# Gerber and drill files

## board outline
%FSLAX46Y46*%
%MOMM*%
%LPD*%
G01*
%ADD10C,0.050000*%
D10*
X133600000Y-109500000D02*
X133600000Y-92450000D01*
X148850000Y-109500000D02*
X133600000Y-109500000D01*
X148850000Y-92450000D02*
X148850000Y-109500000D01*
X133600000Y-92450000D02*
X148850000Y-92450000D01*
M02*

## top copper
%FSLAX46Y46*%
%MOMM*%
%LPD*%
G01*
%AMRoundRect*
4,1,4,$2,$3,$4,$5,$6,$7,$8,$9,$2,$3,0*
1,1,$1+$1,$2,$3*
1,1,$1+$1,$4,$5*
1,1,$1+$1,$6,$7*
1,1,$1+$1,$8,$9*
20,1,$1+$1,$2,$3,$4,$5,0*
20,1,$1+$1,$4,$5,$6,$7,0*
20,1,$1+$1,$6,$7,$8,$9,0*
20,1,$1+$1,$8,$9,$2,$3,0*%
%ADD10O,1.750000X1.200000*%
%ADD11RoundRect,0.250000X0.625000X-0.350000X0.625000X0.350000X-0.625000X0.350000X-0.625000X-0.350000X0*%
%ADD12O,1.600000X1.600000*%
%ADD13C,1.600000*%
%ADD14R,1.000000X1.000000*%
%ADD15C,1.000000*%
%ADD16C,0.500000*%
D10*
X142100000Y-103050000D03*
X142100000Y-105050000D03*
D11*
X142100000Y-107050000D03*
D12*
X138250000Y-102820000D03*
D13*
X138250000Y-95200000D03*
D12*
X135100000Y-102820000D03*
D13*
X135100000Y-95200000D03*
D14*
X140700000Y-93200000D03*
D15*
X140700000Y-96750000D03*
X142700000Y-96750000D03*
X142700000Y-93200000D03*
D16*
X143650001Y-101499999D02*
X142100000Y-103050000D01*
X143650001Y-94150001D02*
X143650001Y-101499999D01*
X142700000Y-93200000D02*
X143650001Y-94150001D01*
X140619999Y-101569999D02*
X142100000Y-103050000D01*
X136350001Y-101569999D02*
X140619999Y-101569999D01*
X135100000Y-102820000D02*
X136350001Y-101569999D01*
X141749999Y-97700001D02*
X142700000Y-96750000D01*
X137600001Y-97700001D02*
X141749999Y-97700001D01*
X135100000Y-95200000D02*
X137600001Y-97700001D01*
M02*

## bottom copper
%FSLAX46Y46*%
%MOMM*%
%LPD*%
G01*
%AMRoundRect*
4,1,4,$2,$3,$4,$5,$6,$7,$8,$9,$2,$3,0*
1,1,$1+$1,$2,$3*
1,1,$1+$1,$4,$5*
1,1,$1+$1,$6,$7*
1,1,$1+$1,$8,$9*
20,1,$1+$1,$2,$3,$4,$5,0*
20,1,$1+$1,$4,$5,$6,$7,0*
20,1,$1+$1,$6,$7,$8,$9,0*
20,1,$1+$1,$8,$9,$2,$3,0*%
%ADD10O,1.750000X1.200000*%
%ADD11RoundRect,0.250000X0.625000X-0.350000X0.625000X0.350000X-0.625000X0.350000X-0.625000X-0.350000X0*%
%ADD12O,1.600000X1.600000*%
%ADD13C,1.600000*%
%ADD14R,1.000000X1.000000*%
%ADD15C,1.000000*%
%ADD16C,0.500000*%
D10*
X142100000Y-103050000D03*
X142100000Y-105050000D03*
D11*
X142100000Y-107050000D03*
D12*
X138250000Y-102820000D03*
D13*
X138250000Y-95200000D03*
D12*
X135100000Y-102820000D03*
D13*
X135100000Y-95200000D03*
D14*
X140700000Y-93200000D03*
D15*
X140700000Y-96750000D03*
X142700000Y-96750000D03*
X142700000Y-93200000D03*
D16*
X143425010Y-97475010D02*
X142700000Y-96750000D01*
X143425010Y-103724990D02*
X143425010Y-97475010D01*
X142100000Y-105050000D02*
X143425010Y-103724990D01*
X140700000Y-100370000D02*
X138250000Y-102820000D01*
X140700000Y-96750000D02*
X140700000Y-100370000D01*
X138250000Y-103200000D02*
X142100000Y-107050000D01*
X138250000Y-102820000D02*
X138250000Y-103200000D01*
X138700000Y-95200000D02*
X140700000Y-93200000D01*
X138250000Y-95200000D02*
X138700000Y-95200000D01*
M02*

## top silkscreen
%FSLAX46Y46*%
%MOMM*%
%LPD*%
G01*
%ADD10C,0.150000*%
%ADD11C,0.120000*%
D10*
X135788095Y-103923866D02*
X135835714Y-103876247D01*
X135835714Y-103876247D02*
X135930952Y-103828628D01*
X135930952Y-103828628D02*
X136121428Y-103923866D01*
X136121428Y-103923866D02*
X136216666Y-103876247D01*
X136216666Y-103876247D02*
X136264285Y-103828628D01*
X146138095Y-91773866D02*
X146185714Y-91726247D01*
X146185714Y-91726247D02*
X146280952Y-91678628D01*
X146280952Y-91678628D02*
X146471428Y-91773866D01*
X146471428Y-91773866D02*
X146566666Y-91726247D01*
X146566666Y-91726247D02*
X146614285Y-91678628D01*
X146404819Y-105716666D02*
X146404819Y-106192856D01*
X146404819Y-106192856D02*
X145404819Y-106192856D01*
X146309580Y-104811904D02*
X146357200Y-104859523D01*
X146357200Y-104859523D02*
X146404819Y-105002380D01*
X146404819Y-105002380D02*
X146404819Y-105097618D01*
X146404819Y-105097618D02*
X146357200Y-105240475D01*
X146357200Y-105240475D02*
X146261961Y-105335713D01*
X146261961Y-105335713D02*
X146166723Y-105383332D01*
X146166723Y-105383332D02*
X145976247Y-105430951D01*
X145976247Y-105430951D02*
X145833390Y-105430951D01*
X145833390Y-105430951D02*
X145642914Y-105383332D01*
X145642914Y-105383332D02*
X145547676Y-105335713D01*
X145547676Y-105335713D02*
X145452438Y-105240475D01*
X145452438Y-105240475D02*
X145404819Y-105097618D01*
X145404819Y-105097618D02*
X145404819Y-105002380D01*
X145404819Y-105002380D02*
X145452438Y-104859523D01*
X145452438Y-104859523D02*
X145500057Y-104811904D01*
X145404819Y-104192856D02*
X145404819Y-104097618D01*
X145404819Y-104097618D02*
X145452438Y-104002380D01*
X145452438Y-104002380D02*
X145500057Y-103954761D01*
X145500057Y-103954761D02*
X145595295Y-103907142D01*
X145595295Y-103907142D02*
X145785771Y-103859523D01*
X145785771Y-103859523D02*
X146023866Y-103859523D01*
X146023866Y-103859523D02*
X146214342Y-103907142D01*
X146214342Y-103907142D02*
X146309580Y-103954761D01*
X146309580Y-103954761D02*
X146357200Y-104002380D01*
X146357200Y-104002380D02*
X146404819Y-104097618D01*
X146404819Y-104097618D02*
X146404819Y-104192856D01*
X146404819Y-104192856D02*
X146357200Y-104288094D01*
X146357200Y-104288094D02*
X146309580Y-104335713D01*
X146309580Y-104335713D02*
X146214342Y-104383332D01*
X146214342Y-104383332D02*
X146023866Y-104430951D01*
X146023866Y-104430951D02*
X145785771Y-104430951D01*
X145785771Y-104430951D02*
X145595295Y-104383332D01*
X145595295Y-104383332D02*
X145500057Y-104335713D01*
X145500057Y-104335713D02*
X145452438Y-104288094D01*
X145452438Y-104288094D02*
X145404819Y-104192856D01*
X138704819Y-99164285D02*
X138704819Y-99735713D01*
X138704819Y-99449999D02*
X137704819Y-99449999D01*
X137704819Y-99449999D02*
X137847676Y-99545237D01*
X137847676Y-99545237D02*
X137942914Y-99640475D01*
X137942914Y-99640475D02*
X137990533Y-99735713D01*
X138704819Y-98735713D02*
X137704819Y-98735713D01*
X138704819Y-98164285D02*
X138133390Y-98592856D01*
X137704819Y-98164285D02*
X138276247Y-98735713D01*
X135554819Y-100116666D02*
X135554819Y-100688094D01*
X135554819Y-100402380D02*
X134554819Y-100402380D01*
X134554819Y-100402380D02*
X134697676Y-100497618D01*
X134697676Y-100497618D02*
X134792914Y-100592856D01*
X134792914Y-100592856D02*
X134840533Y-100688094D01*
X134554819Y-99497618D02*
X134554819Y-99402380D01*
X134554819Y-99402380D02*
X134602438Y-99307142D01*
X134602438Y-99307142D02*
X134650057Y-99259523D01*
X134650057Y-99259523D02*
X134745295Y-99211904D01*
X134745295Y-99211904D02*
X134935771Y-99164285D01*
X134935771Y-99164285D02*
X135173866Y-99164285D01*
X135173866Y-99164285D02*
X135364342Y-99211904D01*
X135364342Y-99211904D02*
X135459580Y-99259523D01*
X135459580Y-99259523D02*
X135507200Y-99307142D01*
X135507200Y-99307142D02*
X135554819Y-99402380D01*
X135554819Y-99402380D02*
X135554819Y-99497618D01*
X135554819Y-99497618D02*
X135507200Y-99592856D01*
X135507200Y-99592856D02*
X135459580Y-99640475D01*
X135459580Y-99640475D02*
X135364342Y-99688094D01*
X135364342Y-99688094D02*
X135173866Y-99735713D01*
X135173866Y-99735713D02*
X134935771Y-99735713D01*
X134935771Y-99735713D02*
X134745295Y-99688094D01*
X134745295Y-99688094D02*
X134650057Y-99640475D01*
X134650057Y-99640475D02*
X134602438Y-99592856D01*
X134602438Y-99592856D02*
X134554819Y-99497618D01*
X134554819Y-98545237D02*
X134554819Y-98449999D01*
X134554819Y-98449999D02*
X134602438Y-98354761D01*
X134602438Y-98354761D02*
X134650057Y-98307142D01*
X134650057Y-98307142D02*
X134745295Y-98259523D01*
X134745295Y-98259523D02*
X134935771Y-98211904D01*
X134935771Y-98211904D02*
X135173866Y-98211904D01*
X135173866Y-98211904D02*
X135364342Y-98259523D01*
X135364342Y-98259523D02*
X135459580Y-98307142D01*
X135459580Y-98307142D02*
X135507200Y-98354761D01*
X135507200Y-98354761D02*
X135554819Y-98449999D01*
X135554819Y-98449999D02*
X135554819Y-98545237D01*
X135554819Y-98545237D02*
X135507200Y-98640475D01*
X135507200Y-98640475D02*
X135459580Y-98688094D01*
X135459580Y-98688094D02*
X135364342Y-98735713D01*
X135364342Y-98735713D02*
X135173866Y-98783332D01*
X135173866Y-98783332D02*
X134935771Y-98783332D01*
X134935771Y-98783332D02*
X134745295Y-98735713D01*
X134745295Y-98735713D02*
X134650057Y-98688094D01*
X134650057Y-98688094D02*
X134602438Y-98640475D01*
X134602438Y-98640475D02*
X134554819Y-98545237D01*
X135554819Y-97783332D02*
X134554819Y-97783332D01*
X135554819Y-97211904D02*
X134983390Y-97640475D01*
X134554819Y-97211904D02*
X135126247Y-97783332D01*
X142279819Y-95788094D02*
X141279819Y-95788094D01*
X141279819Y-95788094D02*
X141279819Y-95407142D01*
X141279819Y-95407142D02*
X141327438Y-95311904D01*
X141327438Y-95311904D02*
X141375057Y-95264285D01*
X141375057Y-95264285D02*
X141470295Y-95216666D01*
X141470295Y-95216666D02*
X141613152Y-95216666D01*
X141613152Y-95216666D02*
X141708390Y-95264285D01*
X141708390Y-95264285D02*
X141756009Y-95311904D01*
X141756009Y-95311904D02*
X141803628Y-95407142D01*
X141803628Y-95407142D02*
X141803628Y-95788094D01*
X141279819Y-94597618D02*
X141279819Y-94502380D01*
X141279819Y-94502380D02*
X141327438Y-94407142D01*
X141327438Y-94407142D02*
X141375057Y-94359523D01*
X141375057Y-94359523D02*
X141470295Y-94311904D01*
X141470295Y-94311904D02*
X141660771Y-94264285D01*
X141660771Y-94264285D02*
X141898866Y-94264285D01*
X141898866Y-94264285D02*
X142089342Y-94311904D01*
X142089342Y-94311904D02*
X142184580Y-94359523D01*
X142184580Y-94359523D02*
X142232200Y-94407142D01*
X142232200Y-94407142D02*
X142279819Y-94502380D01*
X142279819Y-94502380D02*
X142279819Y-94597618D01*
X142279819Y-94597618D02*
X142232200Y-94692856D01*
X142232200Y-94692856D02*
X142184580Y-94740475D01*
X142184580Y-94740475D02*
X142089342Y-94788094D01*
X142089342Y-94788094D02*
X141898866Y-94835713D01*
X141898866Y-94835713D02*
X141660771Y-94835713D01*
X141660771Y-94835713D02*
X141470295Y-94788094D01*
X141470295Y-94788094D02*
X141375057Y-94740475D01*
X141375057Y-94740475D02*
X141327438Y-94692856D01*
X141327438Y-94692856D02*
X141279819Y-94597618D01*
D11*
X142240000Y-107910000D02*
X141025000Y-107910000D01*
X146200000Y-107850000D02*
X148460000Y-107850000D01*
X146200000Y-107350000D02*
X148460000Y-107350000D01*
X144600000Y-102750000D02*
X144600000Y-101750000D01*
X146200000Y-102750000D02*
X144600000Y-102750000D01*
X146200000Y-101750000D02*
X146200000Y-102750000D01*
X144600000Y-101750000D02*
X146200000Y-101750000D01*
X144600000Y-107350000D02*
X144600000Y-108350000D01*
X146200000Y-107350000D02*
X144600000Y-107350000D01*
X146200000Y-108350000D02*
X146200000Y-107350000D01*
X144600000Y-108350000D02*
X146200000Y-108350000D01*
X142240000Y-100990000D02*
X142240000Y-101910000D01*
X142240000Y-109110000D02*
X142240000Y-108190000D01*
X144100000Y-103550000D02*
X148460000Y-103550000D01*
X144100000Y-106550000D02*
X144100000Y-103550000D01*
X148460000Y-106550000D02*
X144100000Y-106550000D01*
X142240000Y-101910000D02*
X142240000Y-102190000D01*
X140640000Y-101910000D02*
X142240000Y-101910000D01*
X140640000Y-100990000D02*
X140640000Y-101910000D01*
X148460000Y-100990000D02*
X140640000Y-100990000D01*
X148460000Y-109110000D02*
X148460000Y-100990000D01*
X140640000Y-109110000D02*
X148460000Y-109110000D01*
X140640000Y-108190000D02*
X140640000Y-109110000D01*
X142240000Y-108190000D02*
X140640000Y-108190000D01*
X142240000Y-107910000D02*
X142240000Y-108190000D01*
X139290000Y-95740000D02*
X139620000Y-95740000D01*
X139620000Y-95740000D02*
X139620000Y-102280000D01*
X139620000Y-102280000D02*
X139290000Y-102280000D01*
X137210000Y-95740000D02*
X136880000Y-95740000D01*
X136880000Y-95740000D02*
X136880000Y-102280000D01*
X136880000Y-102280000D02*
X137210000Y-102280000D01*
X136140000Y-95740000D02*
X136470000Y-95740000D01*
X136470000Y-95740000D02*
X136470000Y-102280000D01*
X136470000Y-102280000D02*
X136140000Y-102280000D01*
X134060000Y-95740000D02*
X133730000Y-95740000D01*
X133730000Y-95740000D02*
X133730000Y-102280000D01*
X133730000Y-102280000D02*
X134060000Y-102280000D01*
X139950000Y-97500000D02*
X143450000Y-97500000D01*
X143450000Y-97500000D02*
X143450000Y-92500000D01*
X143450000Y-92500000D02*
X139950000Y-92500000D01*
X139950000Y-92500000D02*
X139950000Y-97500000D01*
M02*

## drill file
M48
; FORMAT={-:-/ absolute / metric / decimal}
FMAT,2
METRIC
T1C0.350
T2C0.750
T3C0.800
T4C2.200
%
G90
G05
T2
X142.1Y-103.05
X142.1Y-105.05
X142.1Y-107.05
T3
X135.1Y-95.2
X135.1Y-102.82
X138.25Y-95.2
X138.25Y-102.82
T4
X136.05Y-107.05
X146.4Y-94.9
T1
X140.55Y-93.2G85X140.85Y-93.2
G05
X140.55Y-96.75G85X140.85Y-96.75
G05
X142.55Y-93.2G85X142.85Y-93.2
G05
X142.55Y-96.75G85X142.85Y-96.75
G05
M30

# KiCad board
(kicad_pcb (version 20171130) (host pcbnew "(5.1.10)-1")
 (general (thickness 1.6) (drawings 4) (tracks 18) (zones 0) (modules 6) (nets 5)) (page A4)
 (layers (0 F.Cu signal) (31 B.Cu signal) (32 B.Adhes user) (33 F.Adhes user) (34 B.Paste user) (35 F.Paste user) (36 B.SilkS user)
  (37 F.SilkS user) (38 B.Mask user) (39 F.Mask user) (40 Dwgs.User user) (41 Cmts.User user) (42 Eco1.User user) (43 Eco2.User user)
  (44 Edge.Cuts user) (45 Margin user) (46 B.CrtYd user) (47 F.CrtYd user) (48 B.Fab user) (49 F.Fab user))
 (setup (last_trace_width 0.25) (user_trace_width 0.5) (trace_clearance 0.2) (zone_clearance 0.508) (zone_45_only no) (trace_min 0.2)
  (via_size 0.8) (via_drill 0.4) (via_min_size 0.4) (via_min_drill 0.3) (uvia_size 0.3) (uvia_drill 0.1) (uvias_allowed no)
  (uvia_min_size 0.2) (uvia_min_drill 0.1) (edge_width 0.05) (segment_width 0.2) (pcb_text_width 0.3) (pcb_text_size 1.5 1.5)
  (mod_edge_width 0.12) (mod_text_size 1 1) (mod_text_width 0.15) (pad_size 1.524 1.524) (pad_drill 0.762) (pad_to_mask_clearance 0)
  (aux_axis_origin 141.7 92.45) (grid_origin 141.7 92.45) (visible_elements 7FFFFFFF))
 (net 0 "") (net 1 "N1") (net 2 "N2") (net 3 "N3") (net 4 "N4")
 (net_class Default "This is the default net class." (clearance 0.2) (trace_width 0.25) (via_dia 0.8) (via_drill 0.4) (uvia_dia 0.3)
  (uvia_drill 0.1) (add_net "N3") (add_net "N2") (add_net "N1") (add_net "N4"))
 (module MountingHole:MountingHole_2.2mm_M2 (layer F.Cu) (at 136.05 107.05) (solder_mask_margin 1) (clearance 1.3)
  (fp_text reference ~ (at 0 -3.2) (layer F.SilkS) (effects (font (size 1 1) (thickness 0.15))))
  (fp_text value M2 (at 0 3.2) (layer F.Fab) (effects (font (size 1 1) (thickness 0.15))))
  (pad 1 np_thru_hole circle (at 0 0) (size 2.2 2.2) (drill 2.2) (layers *.Cu *.Mask)))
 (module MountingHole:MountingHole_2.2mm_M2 (layer F.Cu) (at 146.4 94.9) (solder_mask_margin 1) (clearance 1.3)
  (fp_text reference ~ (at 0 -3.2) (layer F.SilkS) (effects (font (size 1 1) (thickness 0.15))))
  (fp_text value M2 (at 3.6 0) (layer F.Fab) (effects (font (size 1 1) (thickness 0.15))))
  (pad 1 np_thru_hole circle (at 0 0) (size 2.2 2.2) (drill 2.2) (layers *.Cu *.Mask)))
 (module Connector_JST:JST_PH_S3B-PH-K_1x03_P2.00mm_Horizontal (layer F.Cu) (at 142.1 107.05 90)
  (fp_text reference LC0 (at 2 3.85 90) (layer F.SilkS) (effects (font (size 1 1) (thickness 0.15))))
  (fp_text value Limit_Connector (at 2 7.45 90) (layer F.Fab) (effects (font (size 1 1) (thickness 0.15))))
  (fp_line (start -0.86 0.14) (end -0.86 -1.075) (layer F.SilkS) (width 0.12))
  (fp_line (start -0.8 4.1) (end -0.8 6.36) (layer F.SilkS) (width 0.12))
  (fp_line (start -0.3 4.1) (end -0.3 6.36) (layer F.SilkS) (width 0.12))
  (fp_line (start 4.3 2.5) (end 5.3 2.5) (layer F.SilkS) (width 0.12))
  (fp_line (start 4.3 4.1) (end 4.3 2.5) (layer F.SilkS) (width 0.12))
  (fp_line (start 5.3 4.1) (end 4.3 4.1) (layer F.SilkS) (width 0.12))
  (fp_line (start 5.3 2.5) (end 5.3 4.1) (layer F.SilkS) (width 0.12))
  (fp_line (start -0.3 2.5) (end -1.3 2.5) (layer F.SilkS) (width 0.12))
  (fp_line (start -0.3 4.1) (end -0.3 2.5) (layer F.SilkS) (width 0.12))
  (fp_line (start -1.3 4.1) (end -0.3 4.1) (layer F.SilkS) (width 0.12))
  (fp_line (start -1.3 2.5) (end -1.3 4.1) (layer F.SilkS) (width 0.12))
  (fp_line (start 6.06 0.14) (end 5.14 0.14) (layer F.SilkS) (width 0.12))
  (fp_line (start -2.06 0.14) (end -1.14 0.14) (layer F.SilkS) (width 0.12))
  (fp_line (start 3.5 2) (end 3.5 6.36) (layer F.SilkS) (width 0.12))
  (fp_line (start 0.5 2) (end 3.5 2) (layer F.SilkS) (width 0.12))
  (fp_line (start 0.5 6.36) (end 0.5 2) (layer F.SilkS) (width 0.12))
  (fp_line (start 5.14 0.14) (end 4.86 0.14) (layer F.SilkS) (width 0.12))
  (fp_line (start 5.14 -1.46) (end 5.14 0.14) (layer F.SilkS) (width 0.12))
  (fp_line (start 6.06 -1.46) (end 5.14 -1.46) (layer F.SilkS) (width 0.12))
  (fp_line (start 6.06 6.36) (end 6.06 -1.46) (layer F.SilkS) (width 0.12))
  (fp_line (start -2.06 6.36) (end 6.06 6.36) (layer F.SilkS) (width 0.12))
  (fp_line (start -2.06 -1.46) (end -2.06 6.36) (layer F.SilkS) (width 0.12))
  (fp_line (start -1.14 -1.46) (end -2.06 -1.46) (layer F.SilkS) (width 0.12))
  (fp_line (start -1.14 0.14) (end -1.14 -1.46) (layer F.SilkS) (width 0.12))
  (fp_line (start -0.86 0.14) (end -1.14 0.14) (layer F.SilkS) (width 0.12))
  (pad 3 thru_hole oval (at 4 0 90) (size 1.2 1.75) (drill 0.75) (layers *.Cu *.Mask) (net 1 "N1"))
  (pad 2 thru_hole oval (at 2 0 90) (size 1.2 1.75) (drill 0.75) (layers *.Cu *.Mask) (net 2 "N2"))
  (pad 1 thru_hole roundrect (at 0 0 90) (size 1.2 1.75) (drill 0.75) (layers *.Cu *.Mask) (roundrect_rratio 0.208333) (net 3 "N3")))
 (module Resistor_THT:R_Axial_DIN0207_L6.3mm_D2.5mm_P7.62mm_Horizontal (layer F.Cu) (at 138.25 95.2 270)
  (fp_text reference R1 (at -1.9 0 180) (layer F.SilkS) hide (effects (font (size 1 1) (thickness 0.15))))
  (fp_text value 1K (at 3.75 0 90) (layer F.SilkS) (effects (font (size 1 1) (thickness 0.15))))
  (fp_line (start 0.54 -1.04) (end 0.54 -1.37) (layer F.SilkS) (width 0.12))
  (fp_line (start 0.54 -1.37) (end 7.08 -1.37) (layer F.SilkS) (width 0.12))
  (fp_line (start 7.08 -1.37) (end 7.08 -1.04) (layer F.SilkS) (width 0.12))
  (fp_line (start 0.54 1.04) (end 0.54 1.37) (layer F.SilkS) (width 0.12))
  (fp_line (start 0.54 1.37) (end 7.08 1.37) (layer F.SilkS) (width 0.12))
  (fp_line (start 7.08 1.37) (end 7.08 1.04) (layer F.SilkS) (width 0.12))
  (pad 2 thru_hole oval (at 7.62 0 270) (size 1.6 1.6) (drill 0.8) (layers *.Cu *.Mask) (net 3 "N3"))
  (pad 1 thru_hole circle (at 0 0 270) (size 1.6 1.6) (drill 0.8) (layers *.Cu *.Mask) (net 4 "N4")))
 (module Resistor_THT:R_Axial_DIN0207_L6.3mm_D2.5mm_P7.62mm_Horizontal (layer F.Cu) (at 135.1 95.2 270)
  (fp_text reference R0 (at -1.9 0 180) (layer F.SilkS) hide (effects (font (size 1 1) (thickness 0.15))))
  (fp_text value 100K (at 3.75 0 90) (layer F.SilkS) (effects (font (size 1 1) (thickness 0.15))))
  (fp_line (start 0.54 -1.04) (end 0.54 -1.37) (layer F.SilkS) (width 0.12))
  (fp_line (start 0.54 -1.37) (end 7.08 -1.37) (layer F.SilkS) (width 0.12))
  (fp_line (start 7.08 -1.37) (end 7.08 -1.04) (layer F.SilkS) (width 0.12))
  (fp_line (start 0.54 1.04) (end 0.54 1.37) (layer F.SilkS) (width 0.12))
  (fp_line (start 0.54 1.37) (end 7.08 1.37) (layer F.SilkS) (width 0.12))
  (fp_line (start 7.08 1.37) (end 7.08 1.04) (layer F.SilkS) (width 0.12))
  (pad 2 thru_hole oval (at 7.62 0 270) (size 1.6 1.6) (drill 0.8) (layers *.Cu *.Mask) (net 1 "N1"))
  (pad 1 thru_hole circle (at 0 0 270) (size 1.6 1.6) (drill 0.8) (layers *.Cu *.Mask) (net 2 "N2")))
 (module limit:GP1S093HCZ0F (layer F.Cu) (at 141.7 95 90)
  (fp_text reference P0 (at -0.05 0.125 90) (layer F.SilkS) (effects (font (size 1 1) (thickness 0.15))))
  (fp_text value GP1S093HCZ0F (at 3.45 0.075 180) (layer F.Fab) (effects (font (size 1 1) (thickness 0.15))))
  (fp_line (start -2.5 -1.75) (end -2.5 1.75) (layer F.SilkS) (width 0.12))
  (fp_line (start -2.5 1.75) (end 2.5 1.75) (layer F.SilkS) (width 0.12))
  (fp_line (start 2.5 1.75) (end 2.5 -1.75) (layer F.SilkS) (width 0.12))
  (fp_line (start 2.5 -1.75) (end -2.5 -1.75) (layer F.SilkS) (width 0.12))
  (pad 1 thru_hole rect (at 1.8 -1 90) (size 1 1) (drill oval 0.35 0.65) (layers *.Cu *.Mask) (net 4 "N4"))
  (pad 2 thru_hole circle (at -1.75 -1 90) (size 1 1) (drill oval 0.35 0.65) (layers *.Cu *.Mask) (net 3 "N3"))
  (pad 3 thru_hole circle (at -1.75 1 90) (size 1 1) (drill oval 0.35 0.65) (layers *.Cu *.Mask) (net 2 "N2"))
  (pad 4 thru_hole circle (at 1.8 1 90) (size 1 1) (drill oval 0.35 0.65) (layers *.Cu *.Mask) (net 1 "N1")))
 (gr_line (start 133.6 109.5) (end 133.6 92.45) (layer Edge.Cuts) (width 0.05))
 (gr_line (start 148.85 109.5) (end 133.6 109.5) (layer Edge.Cuts) (width 0.05))
 (gr_line (start 148.85 92.45) (end 148.85 109.5) (layer Edge.Cuts) (width 0.05))
 (gr_line (start 133.6 92.45) (end 148.85 92.45) (layer Edge.Cuts) (width 0.05))
 (segment (start 143.650001 101.499999) (end 142.1 103.05) (width 0.5) (layer F.Cu) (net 1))
 (segment (start 143.650001 94.150001) (end 143.650001 101.499999) (width 0.5) (layer F.Cu) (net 1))
 (segment (start 142.7 93.2) (end 143.650001 94.150001) (width 0.5) (layer F.Cu) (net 1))
 (segment (start 140.619999 101.569999) (end 142.1 103.05) (width 0.5) (layer F.Cu) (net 1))
 (segment (start 136.350001 101.569999) (end 140.619999 101.569999) (width 0.5) (layer F.Cu) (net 1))
 (segment (start 135.1 102.82) (end 136.350001 101.569999) (width 0.5) (layer F.Cu) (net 1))
 (segment (start 143.42501 97.47501) (end 142.7 96.75) (width 0.5) (layer B.Cu) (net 2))
 (segment (start 143.42501 103.72499) (end 143.42501 97.47501) (width 0.5) (layer B.Cu) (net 2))
 (segment (start 142.1 105.05) (end 143.42501 103.72499) (width 0.5) (layer B.Cu) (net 2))
 (segment (start 141.749999 97.700001) (end 142.7 96.75) (width 0.5) (layer F.Cu) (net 2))
 (segment (start 137.600001 97.700001) (end 141.749999 97.700001) (width 0.5) (layer F.Cu) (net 2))
 (segment (start 135.1 95.2) (end 137.600001 97.700001) (width 0.5) (layer F.Cu) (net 2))
 (segment (start 140.7 100.37) (end 138.25 102.82) (width 0.5) (layer B.Cu) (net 3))
 (segment (start 140.7 96.75) (end 140.7 100.37) (width 0.5) (layer B.Cu) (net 3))
 (segment (start 138.25 103.2) (end 142.1 107.05) (width 0.5) (layer B.Cu) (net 3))
 (segment (start 138.25 102.82) (end 138.25 103.2) (width 0.5) (layer B.Cu) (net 3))
 (segment (start 138.7 95.2) (end 140.7 93.2) (width 0.5) (layer B.Cu) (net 4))
 (segment (start 138.25 95.2) (end 138.7 95.2) (width 0.5) (layer B.Cu) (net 4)))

